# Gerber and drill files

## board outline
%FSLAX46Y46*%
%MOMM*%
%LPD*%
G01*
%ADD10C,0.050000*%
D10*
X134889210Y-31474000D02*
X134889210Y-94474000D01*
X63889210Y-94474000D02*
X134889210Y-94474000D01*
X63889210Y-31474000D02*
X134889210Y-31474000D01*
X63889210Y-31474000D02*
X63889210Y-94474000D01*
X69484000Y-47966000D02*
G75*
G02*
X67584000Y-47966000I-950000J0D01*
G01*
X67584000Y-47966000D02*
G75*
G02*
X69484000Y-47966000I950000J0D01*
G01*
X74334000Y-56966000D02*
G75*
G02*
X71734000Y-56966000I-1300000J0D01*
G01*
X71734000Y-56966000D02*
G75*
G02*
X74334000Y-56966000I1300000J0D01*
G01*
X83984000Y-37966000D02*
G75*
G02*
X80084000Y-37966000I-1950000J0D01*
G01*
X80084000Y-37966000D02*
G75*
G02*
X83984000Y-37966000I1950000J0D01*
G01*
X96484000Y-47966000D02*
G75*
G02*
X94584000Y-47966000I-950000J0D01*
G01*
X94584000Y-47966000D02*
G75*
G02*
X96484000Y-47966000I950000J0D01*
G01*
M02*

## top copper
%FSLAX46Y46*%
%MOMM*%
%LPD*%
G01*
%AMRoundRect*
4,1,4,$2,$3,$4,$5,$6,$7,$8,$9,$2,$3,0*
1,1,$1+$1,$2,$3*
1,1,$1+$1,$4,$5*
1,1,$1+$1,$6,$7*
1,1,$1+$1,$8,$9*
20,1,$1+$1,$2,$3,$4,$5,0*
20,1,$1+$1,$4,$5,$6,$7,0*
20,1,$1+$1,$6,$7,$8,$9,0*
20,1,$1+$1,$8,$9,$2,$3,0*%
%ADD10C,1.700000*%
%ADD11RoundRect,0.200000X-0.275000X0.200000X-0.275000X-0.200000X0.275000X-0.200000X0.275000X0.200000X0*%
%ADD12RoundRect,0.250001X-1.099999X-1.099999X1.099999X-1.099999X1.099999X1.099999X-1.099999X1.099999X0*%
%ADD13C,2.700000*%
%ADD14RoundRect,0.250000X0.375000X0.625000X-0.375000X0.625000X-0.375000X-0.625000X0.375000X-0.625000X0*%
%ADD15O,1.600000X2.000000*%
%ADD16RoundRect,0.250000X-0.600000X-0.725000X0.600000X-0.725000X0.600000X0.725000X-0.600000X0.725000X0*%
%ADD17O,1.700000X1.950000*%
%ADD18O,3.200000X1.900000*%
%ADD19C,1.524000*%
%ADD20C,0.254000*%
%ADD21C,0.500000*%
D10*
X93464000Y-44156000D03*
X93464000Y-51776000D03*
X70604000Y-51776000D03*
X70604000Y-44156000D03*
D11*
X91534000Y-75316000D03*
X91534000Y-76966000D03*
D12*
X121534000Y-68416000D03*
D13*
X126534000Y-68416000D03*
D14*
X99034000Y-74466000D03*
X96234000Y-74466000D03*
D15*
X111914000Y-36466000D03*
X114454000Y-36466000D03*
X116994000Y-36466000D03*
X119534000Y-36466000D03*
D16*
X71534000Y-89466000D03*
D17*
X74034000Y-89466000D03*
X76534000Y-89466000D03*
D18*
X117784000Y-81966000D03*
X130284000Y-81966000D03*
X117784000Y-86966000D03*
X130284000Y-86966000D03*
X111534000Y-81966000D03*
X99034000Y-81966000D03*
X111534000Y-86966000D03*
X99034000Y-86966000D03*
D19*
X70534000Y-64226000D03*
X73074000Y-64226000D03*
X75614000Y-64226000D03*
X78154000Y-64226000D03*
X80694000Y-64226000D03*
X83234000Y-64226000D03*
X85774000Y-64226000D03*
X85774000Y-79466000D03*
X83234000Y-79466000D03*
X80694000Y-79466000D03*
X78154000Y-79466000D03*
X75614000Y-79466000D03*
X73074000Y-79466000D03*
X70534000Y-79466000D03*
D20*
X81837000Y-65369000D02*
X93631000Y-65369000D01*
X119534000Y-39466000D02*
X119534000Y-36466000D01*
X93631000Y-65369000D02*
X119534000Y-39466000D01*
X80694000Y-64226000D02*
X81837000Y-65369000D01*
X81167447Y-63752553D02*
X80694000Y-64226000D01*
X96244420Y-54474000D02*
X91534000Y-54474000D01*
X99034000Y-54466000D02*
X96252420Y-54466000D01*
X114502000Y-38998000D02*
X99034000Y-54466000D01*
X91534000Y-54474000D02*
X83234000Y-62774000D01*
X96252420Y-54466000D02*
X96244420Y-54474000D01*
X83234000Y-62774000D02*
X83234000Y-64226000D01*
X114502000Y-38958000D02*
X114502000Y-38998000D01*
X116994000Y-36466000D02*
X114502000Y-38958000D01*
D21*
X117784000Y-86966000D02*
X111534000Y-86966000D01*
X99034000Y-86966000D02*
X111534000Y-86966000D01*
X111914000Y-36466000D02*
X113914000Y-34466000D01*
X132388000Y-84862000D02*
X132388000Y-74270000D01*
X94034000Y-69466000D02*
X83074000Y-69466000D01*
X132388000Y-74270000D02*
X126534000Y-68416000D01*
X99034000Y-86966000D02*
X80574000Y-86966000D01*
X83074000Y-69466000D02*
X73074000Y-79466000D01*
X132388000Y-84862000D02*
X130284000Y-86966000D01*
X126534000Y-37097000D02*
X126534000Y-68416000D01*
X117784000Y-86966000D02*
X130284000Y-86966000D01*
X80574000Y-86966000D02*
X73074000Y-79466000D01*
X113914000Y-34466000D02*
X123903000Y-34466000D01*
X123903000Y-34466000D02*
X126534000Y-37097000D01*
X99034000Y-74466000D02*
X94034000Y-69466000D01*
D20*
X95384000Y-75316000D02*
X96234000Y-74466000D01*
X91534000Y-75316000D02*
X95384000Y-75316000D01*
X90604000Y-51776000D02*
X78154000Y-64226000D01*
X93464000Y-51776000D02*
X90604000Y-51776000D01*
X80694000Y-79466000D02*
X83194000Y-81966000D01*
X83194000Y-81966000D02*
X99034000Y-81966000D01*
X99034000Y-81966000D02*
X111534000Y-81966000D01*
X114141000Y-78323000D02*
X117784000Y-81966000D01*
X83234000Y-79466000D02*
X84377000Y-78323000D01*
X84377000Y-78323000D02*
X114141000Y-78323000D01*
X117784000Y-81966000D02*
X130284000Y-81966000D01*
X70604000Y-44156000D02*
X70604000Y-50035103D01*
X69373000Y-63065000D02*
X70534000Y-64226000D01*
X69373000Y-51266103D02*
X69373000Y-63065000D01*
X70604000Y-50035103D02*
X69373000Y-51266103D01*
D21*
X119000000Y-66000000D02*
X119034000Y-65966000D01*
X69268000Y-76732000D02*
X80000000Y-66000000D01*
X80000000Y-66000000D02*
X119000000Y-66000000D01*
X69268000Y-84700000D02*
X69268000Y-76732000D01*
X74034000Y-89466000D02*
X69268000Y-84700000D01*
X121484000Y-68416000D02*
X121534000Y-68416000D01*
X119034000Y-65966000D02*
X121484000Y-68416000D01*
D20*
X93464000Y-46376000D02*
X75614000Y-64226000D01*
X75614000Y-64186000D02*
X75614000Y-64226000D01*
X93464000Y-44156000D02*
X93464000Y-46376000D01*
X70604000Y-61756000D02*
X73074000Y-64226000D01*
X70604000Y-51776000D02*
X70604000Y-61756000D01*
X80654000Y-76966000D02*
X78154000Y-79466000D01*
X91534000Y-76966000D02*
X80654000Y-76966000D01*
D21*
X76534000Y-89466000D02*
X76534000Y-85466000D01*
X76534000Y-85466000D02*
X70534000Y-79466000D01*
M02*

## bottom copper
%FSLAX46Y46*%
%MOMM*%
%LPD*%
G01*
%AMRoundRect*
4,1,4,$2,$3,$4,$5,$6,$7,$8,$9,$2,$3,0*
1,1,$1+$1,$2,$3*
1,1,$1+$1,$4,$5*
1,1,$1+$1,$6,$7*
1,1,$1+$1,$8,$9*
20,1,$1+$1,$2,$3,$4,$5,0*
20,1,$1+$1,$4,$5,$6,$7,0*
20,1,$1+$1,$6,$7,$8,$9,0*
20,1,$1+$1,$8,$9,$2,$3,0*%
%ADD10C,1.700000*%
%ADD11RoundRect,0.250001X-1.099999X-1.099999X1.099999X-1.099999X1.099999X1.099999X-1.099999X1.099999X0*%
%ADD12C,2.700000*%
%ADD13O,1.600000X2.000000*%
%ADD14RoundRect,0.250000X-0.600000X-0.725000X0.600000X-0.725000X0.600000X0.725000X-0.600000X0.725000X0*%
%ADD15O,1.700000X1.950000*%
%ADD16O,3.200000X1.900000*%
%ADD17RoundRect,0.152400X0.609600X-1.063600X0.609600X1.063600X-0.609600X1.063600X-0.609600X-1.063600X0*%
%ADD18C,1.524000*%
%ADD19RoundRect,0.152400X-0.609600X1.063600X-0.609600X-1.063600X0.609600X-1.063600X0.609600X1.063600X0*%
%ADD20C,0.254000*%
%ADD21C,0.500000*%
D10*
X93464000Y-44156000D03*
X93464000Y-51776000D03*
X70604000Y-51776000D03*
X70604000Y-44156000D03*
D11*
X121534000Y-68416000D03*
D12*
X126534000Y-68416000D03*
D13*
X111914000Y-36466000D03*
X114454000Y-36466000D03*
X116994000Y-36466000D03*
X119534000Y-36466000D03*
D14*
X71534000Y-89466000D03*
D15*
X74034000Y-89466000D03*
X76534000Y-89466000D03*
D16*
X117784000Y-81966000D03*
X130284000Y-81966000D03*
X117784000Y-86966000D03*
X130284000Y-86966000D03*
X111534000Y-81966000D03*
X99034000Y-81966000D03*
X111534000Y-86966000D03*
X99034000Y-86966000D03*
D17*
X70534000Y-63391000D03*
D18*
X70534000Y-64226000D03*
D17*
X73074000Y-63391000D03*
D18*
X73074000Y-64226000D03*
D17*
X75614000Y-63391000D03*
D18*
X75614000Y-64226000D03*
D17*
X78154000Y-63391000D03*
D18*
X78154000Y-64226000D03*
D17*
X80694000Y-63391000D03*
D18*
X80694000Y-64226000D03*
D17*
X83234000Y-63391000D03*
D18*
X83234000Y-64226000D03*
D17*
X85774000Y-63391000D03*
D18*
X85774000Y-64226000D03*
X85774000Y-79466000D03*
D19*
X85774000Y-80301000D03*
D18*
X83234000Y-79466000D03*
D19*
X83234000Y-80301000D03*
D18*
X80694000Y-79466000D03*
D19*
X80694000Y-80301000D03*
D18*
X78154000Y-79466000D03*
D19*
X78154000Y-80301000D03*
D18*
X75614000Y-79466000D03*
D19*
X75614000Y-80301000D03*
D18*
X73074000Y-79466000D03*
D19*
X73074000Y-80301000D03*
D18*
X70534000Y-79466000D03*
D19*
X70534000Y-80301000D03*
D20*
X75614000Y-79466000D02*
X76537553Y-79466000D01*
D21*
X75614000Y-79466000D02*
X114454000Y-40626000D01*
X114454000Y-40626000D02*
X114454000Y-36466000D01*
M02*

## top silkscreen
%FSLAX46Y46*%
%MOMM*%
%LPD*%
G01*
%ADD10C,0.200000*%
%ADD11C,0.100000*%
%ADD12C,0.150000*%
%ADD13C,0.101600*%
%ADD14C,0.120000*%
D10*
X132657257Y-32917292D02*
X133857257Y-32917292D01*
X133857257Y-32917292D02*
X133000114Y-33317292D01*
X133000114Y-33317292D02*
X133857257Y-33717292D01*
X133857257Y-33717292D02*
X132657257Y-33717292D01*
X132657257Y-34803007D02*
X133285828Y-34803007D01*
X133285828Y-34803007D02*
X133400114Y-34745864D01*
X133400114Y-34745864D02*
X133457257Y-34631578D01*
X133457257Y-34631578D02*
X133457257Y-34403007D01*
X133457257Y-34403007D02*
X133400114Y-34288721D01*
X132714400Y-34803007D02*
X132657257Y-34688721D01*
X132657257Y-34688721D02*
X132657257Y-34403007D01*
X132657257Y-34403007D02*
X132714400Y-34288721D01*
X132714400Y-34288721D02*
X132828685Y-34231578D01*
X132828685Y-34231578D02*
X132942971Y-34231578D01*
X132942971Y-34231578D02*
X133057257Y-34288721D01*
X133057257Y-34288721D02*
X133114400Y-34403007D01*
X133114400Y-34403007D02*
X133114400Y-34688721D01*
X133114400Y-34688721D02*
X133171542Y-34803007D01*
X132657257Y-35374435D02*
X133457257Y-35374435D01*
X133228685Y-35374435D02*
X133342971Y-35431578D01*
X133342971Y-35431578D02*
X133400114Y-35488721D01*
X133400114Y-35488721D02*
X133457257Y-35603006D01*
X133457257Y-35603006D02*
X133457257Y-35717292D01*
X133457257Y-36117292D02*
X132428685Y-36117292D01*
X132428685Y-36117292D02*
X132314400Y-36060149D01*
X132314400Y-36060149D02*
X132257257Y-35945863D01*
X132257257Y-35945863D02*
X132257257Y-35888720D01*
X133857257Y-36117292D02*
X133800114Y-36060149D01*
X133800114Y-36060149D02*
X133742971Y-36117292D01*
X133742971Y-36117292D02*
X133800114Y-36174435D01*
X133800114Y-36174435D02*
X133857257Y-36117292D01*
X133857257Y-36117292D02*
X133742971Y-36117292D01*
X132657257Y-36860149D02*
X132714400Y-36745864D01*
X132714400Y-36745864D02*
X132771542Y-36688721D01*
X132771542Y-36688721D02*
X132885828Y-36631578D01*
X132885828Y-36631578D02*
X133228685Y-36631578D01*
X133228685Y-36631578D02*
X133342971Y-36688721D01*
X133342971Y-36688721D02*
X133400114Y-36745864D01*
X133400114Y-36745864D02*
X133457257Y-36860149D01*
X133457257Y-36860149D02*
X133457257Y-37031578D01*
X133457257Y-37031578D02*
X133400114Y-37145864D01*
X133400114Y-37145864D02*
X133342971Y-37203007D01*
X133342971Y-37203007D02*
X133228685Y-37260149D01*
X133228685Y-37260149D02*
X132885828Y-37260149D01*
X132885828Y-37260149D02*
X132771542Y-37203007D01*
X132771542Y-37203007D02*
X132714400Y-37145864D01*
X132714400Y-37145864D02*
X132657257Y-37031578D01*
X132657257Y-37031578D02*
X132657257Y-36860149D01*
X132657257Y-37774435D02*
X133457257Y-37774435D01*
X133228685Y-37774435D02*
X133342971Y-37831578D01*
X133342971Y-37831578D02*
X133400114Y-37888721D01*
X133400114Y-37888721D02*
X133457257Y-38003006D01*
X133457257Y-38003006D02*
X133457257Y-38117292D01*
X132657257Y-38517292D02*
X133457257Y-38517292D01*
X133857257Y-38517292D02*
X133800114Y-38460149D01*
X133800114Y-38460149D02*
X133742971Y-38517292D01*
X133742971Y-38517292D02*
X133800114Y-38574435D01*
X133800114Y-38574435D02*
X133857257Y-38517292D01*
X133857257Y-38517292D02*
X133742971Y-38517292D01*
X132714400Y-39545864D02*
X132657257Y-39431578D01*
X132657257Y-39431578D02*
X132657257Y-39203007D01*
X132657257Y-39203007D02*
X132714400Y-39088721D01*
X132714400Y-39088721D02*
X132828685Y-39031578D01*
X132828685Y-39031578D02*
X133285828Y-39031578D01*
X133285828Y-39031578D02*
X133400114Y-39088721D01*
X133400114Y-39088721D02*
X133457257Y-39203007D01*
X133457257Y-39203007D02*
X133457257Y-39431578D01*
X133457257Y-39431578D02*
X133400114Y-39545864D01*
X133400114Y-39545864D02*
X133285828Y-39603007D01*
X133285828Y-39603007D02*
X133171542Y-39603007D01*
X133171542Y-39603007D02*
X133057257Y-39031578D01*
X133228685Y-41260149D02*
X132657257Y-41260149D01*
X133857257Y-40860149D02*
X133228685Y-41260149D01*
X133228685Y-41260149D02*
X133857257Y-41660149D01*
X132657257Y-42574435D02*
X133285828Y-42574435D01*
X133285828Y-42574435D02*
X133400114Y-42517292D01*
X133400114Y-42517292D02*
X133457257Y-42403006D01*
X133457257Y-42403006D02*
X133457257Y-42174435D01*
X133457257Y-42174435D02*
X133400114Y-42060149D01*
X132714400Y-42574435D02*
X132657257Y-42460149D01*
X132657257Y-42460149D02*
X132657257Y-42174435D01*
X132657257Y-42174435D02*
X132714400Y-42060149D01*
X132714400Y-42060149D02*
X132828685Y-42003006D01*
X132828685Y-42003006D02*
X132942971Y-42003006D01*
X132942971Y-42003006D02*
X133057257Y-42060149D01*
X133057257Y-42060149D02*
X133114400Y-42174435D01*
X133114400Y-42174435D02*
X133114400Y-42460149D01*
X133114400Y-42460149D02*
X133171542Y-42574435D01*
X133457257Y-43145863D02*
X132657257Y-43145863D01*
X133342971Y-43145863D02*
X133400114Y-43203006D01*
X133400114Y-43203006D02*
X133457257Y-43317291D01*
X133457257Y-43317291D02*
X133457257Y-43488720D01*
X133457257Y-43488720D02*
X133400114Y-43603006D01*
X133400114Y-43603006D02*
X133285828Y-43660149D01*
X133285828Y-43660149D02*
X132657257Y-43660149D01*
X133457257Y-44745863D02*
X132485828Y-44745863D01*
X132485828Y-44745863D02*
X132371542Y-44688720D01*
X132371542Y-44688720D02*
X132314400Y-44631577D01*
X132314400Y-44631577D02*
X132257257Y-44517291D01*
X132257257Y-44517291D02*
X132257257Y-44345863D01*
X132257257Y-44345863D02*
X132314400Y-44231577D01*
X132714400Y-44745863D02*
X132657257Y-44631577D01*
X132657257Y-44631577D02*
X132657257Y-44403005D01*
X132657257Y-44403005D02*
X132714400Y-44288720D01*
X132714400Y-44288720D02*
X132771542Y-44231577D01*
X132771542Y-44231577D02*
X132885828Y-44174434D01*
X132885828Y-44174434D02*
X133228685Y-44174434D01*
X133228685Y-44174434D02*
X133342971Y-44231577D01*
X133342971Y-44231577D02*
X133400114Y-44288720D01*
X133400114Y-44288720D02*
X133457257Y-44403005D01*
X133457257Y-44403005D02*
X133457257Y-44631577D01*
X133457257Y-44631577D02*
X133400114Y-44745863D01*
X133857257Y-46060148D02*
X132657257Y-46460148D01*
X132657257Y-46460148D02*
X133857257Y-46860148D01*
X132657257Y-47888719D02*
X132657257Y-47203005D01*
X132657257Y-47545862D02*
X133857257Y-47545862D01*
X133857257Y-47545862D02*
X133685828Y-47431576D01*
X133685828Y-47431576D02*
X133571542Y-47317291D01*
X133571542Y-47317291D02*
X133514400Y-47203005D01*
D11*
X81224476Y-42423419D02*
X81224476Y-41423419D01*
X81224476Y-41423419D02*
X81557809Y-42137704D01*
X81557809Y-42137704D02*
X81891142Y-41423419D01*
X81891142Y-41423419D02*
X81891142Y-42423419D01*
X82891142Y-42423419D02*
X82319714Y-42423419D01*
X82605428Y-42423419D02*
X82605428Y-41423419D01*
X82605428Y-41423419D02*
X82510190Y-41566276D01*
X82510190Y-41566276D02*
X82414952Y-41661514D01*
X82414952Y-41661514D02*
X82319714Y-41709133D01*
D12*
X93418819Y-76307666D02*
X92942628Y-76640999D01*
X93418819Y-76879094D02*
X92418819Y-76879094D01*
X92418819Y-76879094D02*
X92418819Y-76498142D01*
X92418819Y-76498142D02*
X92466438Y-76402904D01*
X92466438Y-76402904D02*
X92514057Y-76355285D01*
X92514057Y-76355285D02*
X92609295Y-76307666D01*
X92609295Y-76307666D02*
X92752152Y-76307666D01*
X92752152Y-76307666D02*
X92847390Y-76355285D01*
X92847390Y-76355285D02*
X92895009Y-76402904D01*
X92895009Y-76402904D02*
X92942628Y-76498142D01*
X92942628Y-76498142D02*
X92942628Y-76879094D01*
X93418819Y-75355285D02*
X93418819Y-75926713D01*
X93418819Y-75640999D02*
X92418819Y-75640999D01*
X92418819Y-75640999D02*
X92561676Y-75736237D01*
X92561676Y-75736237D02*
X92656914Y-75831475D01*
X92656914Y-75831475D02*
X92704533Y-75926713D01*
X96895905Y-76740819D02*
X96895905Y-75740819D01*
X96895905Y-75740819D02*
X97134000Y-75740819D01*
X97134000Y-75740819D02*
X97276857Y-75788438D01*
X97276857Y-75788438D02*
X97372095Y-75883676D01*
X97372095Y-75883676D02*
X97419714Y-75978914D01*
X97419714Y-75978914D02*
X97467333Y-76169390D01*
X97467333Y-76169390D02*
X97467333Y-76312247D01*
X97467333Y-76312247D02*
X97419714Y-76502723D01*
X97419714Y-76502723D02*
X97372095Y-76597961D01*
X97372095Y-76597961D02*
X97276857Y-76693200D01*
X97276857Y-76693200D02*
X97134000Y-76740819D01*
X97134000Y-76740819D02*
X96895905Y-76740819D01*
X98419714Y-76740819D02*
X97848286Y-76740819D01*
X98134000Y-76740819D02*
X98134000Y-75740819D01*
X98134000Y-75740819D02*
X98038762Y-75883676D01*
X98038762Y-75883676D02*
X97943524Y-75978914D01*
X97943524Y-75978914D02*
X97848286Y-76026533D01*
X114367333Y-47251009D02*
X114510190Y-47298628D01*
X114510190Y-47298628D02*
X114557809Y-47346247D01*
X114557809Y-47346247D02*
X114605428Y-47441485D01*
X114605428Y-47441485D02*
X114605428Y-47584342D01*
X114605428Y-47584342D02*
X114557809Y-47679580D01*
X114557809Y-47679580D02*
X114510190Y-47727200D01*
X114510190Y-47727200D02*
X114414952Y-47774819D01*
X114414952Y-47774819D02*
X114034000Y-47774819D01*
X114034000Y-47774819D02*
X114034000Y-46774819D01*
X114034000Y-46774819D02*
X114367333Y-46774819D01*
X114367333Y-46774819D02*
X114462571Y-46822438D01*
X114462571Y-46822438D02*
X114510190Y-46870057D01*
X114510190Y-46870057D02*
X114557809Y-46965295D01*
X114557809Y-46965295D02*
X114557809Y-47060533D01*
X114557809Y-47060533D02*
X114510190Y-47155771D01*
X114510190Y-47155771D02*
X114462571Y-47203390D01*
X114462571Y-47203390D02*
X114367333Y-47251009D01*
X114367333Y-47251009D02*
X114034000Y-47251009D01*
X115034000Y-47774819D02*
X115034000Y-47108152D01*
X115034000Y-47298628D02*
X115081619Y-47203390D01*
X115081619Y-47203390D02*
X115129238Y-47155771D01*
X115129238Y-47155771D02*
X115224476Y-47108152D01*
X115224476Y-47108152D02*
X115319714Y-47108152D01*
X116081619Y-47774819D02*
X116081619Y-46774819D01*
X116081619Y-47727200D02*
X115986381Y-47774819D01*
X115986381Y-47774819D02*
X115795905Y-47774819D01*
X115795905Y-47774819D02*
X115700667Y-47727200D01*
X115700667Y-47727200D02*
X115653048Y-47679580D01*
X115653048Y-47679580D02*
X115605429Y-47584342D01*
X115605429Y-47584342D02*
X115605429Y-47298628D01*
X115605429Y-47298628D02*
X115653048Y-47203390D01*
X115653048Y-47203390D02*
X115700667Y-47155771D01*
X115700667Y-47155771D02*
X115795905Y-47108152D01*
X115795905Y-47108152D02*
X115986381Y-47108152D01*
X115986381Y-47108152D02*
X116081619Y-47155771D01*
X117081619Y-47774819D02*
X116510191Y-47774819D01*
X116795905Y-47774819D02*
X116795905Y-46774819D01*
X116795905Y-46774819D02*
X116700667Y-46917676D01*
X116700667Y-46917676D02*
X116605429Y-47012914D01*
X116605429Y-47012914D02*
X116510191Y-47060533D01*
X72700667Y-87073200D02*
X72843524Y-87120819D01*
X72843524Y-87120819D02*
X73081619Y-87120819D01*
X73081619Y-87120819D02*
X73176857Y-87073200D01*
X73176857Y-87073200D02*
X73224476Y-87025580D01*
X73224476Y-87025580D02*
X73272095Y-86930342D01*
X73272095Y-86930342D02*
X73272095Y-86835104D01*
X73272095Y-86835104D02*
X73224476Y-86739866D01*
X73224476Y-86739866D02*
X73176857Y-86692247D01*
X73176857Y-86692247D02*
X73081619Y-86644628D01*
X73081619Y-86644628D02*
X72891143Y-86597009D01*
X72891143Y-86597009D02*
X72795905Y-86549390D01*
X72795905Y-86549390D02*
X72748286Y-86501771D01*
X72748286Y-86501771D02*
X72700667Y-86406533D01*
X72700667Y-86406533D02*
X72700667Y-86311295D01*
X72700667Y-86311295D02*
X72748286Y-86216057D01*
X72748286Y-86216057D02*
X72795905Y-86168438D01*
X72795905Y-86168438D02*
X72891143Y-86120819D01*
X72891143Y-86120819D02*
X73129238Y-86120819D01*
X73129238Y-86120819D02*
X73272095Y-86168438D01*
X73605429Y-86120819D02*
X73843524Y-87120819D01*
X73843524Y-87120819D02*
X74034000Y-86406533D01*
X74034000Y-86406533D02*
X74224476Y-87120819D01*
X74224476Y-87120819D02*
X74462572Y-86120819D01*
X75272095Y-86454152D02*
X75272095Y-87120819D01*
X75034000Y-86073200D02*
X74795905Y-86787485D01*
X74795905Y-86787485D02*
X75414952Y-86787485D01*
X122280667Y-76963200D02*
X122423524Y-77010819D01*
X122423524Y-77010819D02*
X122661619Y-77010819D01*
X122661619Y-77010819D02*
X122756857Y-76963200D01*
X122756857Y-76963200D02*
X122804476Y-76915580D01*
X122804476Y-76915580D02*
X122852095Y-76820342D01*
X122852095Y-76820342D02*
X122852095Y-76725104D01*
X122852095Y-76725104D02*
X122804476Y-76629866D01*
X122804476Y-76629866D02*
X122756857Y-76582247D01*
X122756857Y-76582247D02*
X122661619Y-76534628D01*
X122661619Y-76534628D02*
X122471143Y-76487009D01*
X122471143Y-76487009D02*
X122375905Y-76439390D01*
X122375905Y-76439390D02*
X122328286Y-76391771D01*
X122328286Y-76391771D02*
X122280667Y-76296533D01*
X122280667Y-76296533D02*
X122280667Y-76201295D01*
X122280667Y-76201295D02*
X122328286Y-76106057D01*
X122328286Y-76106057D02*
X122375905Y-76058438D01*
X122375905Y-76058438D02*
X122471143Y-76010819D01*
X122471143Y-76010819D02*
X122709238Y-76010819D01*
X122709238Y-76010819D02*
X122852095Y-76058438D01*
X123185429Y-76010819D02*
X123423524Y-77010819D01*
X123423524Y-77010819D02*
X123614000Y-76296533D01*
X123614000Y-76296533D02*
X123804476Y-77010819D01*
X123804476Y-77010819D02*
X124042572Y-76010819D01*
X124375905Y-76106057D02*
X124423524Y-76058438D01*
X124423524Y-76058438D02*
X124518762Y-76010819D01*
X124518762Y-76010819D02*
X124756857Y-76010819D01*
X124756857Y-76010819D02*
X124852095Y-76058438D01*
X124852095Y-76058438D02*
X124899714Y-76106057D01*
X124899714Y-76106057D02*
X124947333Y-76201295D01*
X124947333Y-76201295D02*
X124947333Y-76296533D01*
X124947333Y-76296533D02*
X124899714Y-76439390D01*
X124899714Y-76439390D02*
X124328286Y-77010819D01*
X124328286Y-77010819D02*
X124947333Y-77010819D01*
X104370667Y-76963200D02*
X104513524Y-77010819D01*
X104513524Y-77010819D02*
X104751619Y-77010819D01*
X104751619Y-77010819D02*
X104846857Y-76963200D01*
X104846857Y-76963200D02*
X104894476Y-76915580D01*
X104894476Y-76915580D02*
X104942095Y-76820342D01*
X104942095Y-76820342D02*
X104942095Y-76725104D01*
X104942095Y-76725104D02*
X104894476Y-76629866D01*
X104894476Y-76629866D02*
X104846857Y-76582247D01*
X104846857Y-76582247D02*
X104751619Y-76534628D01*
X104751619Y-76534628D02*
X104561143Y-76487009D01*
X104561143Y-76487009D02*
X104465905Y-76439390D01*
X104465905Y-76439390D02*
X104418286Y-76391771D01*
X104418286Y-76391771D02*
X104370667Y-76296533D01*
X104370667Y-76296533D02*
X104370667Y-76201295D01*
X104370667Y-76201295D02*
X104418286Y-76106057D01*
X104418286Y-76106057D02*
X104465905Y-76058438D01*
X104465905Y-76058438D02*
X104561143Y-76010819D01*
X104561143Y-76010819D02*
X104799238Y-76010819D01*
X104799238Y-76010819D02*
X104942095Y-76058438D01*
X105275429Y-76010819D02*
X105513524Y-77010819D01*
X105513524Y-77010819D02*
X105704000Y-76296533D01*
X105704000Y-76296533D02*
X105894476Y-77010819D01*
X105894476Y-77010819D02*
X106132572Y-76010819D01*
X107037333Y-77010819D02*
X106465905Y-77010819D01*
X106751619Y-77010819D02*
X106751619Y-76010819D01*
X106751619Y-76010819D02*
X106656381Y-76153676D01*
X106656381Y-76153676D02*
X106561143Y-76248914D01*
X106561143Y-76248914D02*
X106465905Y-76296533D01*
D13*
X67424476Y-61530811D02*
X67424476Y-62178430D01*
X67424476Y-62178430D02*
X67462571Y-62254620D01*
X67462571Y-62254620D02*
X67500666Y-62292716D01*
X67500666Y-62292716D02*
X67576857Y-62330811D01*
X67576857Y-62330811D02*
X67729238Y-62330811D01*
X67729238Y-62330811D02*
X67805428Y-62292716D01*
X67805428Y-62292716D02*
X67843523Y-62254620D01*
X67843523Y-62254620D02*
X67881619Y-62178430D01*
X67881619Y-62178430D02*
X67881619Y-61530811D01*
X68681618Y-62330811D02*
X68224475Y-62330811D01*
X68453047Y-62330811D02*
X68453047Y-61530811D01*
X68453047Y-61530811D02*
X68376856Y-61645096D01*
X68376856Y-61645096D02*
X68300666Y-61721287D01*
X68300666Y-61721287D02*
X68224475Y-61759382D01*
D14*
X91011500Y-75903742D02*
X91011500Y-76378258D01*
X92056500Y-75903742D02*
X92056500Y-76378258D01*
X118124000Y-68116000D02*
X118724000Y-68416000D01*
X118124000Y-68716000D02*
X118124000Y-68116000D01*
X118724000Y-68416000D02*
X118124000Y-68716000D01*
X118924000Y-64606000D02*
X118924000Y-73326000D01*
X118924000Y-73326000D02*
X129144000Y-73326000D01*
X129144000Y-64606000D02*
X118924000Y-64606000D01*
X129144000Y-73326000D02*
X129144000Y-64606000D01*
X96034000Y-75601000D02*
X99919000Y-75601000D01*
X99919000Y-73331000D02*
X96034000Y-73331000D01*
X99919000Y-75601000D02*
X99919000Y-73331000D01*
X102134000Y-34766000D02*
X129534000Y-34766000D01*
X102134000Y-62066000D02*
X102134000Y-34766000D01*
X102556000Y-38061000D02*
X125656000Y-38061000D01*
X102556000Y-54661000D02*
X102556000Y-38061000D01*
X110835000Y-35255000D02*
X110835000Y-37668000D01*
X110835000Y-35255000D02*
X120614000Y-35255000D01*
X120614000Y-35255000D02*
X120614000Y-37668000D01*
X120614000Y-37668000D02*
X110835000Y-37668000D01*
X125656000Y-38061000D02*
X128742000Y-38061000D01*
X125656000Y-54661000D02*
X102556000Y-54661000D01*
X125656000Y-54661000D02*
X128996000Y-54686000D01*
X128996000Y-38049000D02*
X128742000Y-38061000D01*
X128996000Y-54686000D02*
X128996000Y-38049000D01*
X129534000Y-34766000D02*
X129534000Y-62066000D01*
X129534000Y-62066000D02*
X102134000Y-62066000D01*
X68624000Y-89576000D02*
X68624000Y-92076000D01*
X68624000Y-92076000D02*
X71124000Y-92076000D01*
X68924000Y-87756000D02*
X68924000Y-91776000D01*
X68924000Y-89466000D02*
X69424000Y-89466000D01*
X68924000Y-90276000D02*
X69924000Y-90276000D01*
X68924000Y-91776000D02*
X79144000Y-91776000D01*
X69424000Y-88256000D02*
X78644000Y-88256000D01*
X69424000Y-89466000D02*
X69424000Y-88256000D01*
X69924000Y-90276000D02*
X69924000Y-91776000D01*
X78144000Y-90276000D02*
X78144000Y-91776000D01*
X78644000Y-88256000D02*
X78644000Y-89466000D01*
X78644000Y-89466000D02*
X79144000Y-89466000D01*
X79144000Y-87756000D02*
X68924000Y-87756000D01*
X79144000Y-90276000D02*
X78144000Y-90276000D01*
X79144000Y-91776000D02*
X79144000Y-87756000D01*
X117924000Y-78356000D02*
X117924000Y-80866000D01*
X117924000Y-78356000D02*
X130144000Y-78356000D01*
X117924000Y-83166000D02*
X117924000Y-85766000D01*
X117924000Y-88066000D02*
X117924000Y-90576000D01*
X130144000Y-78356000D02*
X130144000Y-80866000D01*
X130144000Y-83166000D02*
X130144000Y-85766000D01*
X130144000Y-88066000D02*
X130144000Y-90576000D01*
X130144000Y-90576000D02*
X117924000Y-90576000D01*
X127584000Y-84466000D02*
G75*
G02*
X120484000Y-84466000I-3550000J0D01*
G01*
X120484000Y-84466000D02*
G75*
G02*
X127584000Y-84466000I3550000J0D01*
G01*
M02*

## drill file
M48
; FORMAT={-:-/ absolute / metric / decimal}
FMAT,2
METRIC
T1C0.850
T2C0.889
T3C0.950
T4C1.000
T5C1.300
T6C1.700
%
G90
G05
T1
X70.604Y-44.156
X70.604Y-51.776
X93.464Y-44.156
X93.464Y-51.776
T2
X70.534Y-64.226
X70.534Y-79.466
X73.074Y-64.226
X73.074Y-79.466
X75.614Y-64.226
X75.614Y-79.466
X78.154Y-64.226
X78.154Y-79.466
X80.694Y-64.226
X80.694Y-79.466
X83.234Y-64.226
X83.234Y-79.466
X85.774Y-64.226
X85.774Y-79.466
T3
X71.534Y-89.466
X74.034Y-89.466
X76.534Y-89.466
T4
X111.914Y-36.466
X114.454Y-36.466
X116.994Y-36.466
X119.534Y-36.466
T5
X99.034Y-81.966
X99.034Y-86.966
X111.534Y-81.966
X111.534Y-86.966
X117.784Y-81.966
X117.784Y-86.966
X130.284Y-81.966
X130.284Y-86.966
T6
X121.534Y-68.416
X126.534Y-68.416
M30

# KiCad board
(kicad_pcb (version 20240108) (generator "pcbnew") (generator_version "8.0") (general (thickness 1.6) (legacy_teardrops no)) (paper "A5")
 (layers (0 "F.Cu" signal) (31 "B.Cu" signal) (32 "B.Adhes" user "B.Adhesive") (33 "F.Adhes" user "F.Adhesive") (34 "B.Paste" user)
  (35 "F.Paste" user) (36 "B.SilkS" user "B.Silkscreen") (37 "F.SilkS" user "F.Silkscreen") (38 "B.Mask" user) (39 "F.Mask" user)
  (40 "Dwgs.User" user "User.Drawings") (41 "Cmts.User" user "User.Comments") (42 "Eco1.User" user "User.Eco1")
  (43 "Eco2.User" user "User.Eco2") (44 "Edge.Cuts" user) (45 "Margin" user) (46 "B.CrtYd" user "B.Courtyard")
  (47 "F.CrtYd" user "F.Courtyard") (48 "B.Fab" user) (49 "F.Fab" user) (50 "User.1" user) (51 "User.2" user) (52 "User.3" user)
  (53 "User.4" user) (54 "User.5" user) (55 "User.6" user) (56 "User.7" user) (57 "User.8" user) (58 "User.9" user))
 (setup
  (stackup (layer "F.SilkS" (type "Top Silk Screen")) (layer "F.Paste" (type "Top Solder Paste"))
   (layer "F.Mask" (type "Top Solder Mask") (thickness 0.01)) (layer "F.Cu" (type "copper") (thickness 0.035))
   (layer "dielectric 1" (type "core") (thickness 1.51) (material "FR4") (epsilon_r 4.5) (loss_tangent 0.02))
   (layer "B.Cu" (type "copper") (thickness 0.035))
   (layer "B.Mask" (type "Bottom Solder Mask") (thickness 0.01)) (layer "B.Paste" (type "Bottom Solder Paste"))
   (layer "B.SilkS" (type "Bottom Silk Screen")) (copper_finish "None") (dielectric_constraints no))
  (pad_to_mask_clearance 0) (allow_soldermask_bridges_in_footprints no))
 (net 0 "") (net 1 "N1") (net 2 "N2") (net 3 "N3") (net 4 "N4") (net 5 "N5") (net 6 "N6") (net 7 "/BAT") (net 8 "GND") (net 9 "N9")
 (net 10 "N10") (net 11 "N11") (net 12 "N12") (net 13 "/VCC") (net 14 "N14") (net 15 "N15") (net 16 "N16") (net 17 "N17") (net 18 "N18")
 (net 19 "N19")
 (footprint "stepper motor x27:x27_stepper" (layer "F.Cu") (at 84.574 58.126)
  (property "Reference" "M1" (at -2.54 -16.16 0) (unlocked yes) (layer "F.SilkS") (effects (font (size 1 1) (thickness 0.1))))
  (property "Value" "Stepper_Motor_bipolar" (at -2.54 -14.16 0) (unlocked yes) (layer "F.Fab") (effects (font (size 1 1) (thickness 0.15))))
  (fp_circle (center -16.04 -10.16) (end -15.09 -10.16) (stroke (width 0.05) (type default)) (fill none) (layer "Edge.Cuts"))
  (fp_circle (center -11.54 -1.16) (end -10.24 -1.16) (stroke (width 0.05) (type default)) (fill none) (layer "Edge.Cuts"))
  (fp_circle (center -2.54 -20.16) (end -0.59 -20.16) (stroke (width 0.05) (type default)) (fill none) (layer "Edge.Cuts"))
  (fp_circle (center 10.96 -10.16) (end 11.91 -10.16) (stroke (width 0.05) (type default)) (fill none) (layer "Edge.Cuts"))
  (pad "1" thru_hole circle (at 8.89 -13.97) (size 1.7 1.7) (drill 0.85) (layers "*.Cu" "*.Mask") (remove_unused_layers no) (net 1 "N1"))
  (pad "2" thru_hole circle (at 8.89 -6.35) (size 1.7 1.7) (drill 0.85) (layers "*.Cu" "*.Mask") (remove_unused_layers no) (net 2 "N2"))
  (pad "3" thru_hole circle (at -13.97 -6.35) (size 1.7 1.7) (drill 0.85) (layers "*.Cu" "*.Mask") (remove_unused_layers no) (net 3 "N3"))
  (pad "4" thru_hole circle (at -13.97 -13.97) (size 1.7 1.7) (drill 0.85) (layers "*.Cu" "*.Mask") (remove_unused_layers no) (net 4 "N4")))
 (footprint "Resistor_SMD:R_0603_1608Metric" (layer "F.Cu") (at 91.534 76.141 -90)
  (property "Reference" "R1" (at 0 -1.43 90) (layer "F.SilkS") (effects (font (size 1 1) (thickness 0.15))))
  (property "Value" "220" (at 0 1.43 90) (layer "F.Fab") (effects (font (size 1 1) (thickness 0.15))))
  (fp_line (start -0.237258 0.5225) (end 0.237258 0.5225) (stroke (width 0.12) (type solid)) (layer "F.SilkS"))
  (fp_line (start -0.237258 -0.5225) (end 0.237258 -0.5225) (stroke (width 0.12) (type solid)) (layer "F.SilkS"))
  (pad "1" smd roundrect (at -0.825 0 270) (size 0.8 0.95) (layers "F.Cu" "F.Paste" "F.Mask") (roundrect_rratio 0.25) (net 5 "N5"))
  (pad "2" smd roundrect (at 0.825 0 270) (size 0.8 0.95) (layers "F.Cu" "F.Paste" "F.Mask") (roundrect_rratio 0.25) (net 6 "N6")))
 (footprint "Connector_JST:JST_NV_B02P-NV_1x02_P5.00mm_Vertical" (layer "F.Cu") (at 121.534 68.416)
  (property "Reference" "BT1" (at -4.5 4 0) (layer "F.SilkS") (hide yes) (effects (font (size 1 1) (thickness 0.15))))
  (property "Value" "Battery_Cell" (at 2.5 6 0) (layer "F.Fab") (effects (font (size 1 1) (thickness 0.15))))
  (fp_line (start -3.41 -0.3) (end -2.81 0) (stroke (width 0.12) (type solid)) (layer "F.SilkS"))
  (fp_line (start -3.41 0.3) (end -3.41 -0.3) (stroke (width 0.12) (type solid)) (layer "F.SilkS"))
  (fp_line (start -2.81 0) (end -3.41 0.3) (stroke (width 0.12) (type solid)) (layer "F.SilkS"))
  (fp_line (start -2.61 -3.81) (end -2.61 4.91) (stroke (width 0.12) (type solid)) (layer "F.SilkS"))
  (fp_line (start -2.61 4.91) (end 7.61 4.91) (stroke (width 0.12) (type solid)) (layer "F.SilkS"))
  (fp_line (start 7.61 -3.81) (end -2.61 -3.81) (stroke (width 0.12) (type solid)) (layer "F.SilkS"))
  (fp_line (start 7.61 4.91) (end 7.61 -3.81) (stroke (width 0.12) (type solid)) (layer "F.SilkS"))
  (pad "1" thru_hole roundrect (at 0 0) (size 2.7 2.7) (drill 1.7) (layers "*.Cu" "*.Mask") (remove_unused_layers no)
   (roundrect_rratio 0.092593) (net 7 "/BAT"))
  (pad "2" thru_hole circle (at 5 0) (size 2.7 2.7) (drill 1.7) (layers "*.Cu" "*.Mask") (remove_unused_layers no) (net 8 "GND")))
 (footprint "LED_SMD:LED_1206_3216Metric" (layer "F.Cu") (at 97.634 74.466 180)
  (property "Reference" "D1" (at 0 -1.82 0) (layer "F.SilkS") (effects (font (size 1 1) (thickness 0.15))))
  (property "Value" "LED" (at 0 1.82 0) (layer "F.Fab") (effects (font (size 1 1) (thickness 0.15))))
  (fp_line (start 1.6 -1.135) (end -2.285 -1.135) (stroke (width 0.12) (type solid)) (layer "F.SilkS"))
  (fp_line (start -2.285 1.135) (end 1.6 1.135) (stroke (width 0.12) (type solid)) (layer "F.SilkS"))
  (fp_line (start -2.285 -1.135) (end -2.285 1.135) (stroke (width 0.12) (type solid)) (layer "F.SilkS"))
  (pad "1" smd roundrect (at -1.4 0 180) (size 1.25 1.75) (layers "F.Cu" "F.Paste" "F.Mask") (roundrect_rratio 0.2) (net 8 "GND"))
  (pad "2" smd roundrect (at 1.4 0 180) (size 1.25 1.75) (layers "F.Cu" "F.Paste" "F.Mask") (roundrect_rratio 0.2) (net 5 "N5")))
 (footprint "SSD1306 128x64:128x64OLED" (layer "F.Cu") (at 115.534 47.066)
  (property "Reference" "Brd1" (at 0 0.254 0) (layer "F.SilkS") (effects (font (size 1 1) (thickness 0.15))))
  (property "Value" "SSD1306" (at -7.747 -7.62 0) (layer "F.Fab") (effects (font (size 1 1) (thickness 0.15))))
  (fp_line (start -13.4 -12.3) (end 14 -12.3) (stroke (width 0.12) (type solid)) (layer "F.SilkS"))
  (fp_line (start -13.4 15) (end -13.4 -12.3) (stroke (width 0.12) (type solid)) (layer "F.SilkS"))
  (fp_line (start -12.978 -9.005) (end 10.122 -9.005) (stroke (width 0.12) (type solid)) (layer "F.SilkS"))
  (fp_line (start -12.978 7.595) (end -12.978 -9.005) (stroke (width 0.12) (type solid)) (layer "F.SilkS"))
  (fp_line (start -4.699 -11.811) (end -4.699 -9.398) (stroke (width 0.12) (type solid)) (layer "F.SilkS"))
  (fp_line (start -4.699 -11.811) (end 5.08 -11.811) (stroke (width 0.12) (type solid)) (layer "F.SilkS"))
  (fp_line (start 5.08 -11.811) (end 5.08 -9.398) (stroke (width 0.12) (type solid)) (layer "F.SilkS"))
  (fp_line (start 5.08 -9.398) (end -4.699 -9.398) (stroke (width 0.12) (type solid)) (layer "F.SilkS"))
  (fp_line (start 10.122 -9.005) (end 13.208 -9.005) (stroke (width 0.12) (type solid)) (layer "F.SilkS"))
  (fp_line (start 10.122 7.595) (end -12.978 7.595) (stroke (width 0.12) (type solid)) (layer "F.SilkS"))
  (fp_line (start 10.122 7.595) (end 13.462 7.62) (stroke (width 0.12) (type solid)) (layer "F.SilkS"))
  (fp_line (start 13.462 -9.017) (end 13.208 -9.005) (stroke (width 0.12) (type solid)) (layer "F.SilkS"))
  (fp_line (start 13.462 7.62) (end 13.462 -9.017) (stroke (width 0.12) (type solid)) (layer "F.SilkS"))
  (fp_line (start 14 -12.3) (end 14 15) (stroke (width 0.12) (type solid)) (layer "F.SilkS"))
  (fp_line (start 14 15) (end -13.4 15) (stroke (width 0.12) (type solid)) (layer "F.SilkS"))
  (pad "1" thru_hole oval (at -3.62 -10.6 90) (size 2 1.6) (drill 1) (layers "*.Cu" "*.Mask") (remove_unused_layers no) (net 8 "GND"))
  (pad "2" thru_hole oval (at -1.08 -10.6 90) (size 2 1.6) (drill 1) (layers "*.Cu" "*.Mask") (remove_unused_layers no) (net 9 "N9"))
  (pad "3" thru_hole oval (at 1.46 -10.6 90) (size 2 1.6) (drill 1) (layers "*.Cu" "*.Mask") (remove_unused_layers no) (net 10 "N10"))
  (pad "4" thru_hole oval (at 4 -10.6 90) (size 2 1.6) (drill 1) (layers "*.Cu" "*.Mask") (remove_unused_layers no) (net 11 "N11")))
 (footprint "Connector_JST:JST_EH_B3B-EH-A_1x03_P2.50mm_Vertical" (layer "F.Cu") (at 71.534 89.466)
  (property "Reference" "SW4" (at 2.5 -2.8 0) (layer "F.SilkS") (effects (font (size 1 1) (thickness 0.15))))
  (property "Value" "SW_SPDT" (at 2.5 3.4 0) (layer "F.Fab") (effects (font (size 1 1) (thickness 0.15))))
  (fp_line (start -2.91 0.11) (end -2.91 2.61) (stroke (width 0.12) (type solid)) (layer "F.SilkS"))
  (fp_line (start -2.91 2.61) (end -0.41 2.61) (stroke (width 0.12) (type solid)) (layer "F.SilkS"))
  (fp_line (start -2.61 -1.71) (end -2.61 2.31) (stroke (width 0.12) (type solid)) (layer "F.SilkS"))
  (fp_line (start -2.61 0) (end -2.11 0) (stroke (width 0.12) (type solid)) (layer "F.SilkS"))
  (fp_line (start -2.61 0.81) (end -1.61 0.81) (stroke (width 0.12) (type solid)) (layer "F.SilkS"))
  (fp_line (start -2.61 2.31) (end 7.61 2.31) (stroke (width 0.12) (type solid)) (layer "F.SilkS"))
  (fp_line (start -2.11 -1.21) (end 7.11 -1.21) (stroke (width 0.12) (type solid)) (layer "F.SilkS"))
  (fp_line (start -2.11 0) (end -2.11 -1.21) (stroke (width 0.12) (type solid)) (layer "F.SilkS"))
  (fp_line (start -1.61 0.81) (end -1.61 2.31) (stroke (width 0.12) (type solid)) (layer "F.SilkS"))
  (fp_line (start 6.61 0.81) (end 6.61 2.31) (stroke (width 0.12) (type solid)) (layer "F.SilkS"))
  (fp_line (start 7.11 -1.21) (end 7.11 0) (stroke (width 0.12) (type solid)) (layer "F.SilkS"))
  (fp_line (start 7.11 0) (end 7.61 0) (stroke (width 0.12) (type solid)) (layer "F.SilkS"))
  (fp_line (start 7.61 -1.71) (end -2.61 -1.71) (stroke (width 0.12) (type solid)) (layer "F.SilkS"))
  (fp_line (start 7.61 0.81) (end 6.61 0.81) (stroke (width 0.12) (type solid)) (layer "F.SilkS"))
  (fp_line (start 7.61 2.31) (end 7.61 -1.71) (stroke (width 0.12) (type solid)) (layer "F.SilkS"))
  (pad "1" thru_hole roundrect (at 0 0) (size 1.7 1.95) (drill 0.95) (layers "*.Cu" "*.Mask") (remove_unused_layers no)
   (roundrect_rratio 0.147059) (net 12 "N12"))
  (pad "2" thru_hole oval (at 2.5 0) (size 1.7 1.95) (drill 0.95) (layers "*.Cu" "*.Mask") (remove_unused_layers no) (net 7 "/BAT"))
  (pad "3" thru_hole oval (at 5 0) (size 1.7 1.95) (drill 0.95) (layers "*.Cu" "*.Mask") (remove_unused_layers no) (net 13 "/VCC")))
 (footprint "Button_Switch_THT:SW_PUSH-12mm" (layer "F.Cu") (at 117.784 81.966)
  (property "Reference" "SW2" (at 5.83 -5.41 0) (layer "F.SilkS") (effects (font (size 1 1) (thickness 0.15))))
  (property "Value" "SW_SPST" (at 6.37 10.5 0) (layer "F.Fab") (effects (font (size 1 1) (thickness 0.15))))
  (fp_line (start 0.14 -3.61) (end 0.14 -1.1) (stroke (width 0.12) (type default)) (layer "F.SilkS"))
  (fp_line (start 0.14 -3.61) (end 12.36 -3.61) (stroke (width 0.12) (type default)) (layer "F.SilkS"))
  (fp_line (start 0.14 1.2) (end 0.14 3.8) (stroke (width 0.12) (type default)) (layer "F.SilkS"))
  (fp_line (start 0.14 6.1) (end 0.14 8.61) (stroke (width 0.12) (type default)) (layer "F.SilkS"))
  (fp_line (start 12.36 -3.61) (end 12.36 -1.1) (stroke (width 0.12) (type default)) (layer "F.SilkS"))
  (fp_line (start 12.36 1.2) (end 12.36 3.8) (stroke (width 0.12) (type default)) (layer "F.SilkS"))
  (fp_line (start 12.36 6.1) (end 12.36 8.61) (stroke (width 0.12) (type default)) (layer "F.SilkS"))
  (fp_line (start 12.36 8.61) (end 0.14 8.61) (stroke (width 0.12) (type default)) (layer "F.SilkS"))
  (fp_circle (center 6.25 2.5) (end 9.8 2.5) (stroke (width 0.12) (type default)) (fill none) (layer "F.SilkS"))
  (pad "1" thru_hole oval (at 0 0) (size 3.2 1.9) (drill 1.3) (layers "*.Cu" "*.Mask") (remove_unused_layers no) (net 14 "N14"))
  (pad "1" thru_hole oval (at 12.5 0) (size 3.2 1.9) (drill 1.3) (layers "*.Cu" "*.Mask") (remove_unused_layers no) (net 14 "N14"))
  (pad "2" thru_hole oval (at 0 5) (size 3.2 1.9) (drill 1.3) (layers "*.Cu" "*.Mask") (remove_unused_layers no) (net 8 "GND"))
  (pad "2" thru_hole oval (at 12.5 5) (size 3.2 1.9) (drill 1.3) (layers "*.Cu" "*.Mask") (remove_unused_layers no) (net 8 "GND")))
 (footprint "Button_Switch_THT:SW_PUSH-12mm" (layer "B.Cu") (at 111.534 81.966 180)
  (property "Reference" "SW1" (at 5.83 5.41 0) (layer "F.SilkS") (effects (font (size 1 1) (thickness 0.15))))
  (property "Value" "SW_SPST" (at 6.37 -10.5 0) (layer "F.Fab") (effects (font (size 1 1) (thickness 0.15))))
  (pad "1" thru_hole oval (at 0 0 180) (size 3.2 1.9) (drill 1.3) (layers "*.Cu" "*.Mask") (remove_unused_layers no) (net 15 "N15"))
  (pad "1" thru_hole oval (at 12.5 0 180) (size 3.2 1.9) (drill 1.3) (layers "*.Cu" "*.Mask") (remove_unused_layers no) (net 15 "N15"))
  (pad "2" thru_hole oval (at 0 -5 180) (size 3.2 1.9) (drill 1.3) (layers "*.Cu" "*.Mask") (remove_unused_layers no) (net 8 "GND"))
  (pad "2" thru_hole oval (at 12.5 -5 180) (size 3.2 1.9) (drill 1.3) (layers "*.Cu" "*.Mask") (remove_unused_layers no) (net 8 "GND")))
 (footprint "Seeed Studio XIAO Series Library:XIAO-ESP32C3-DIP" (layer "B.Cu") (at 78.154 71.966 -90)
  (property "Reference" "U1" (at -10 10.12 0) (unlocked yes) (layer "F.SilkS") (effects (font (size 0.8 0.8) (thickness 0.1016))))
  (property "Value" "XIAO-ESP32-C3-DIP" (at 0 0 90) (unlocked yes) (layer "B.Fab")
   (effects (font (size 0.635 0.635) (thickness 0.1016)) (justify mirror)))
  (pad "1" smd roundrect (at -8.575 7.62 90) (size 2.432 1.524) (layers "B.Cu" "B.Mask") (roundrect_rratio 0.1) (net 4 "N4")
   (thermal_bridge_angle 45))
  (pad "1" thru_hole circle (at -7.74 7.62 90) (size 1.524 1.524) (drill 0.889) (layers "*.Cu" "*.Mask") (remove_unused_layers no)
   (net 4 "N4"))
  (pad "2" smd roundrect (at -8.575 5.08 90) (size 2.432 1.524) (layers "B.Cu" "B.Mask") (roundrect_rratio 0.1) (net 3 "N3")
   (thermal_bridge_angle 45))
  (pad "2" thru_hole circle (at -7.74 5.08 90) (size 1.524 1.524) (drill 0.889) (layers "*.Cu" "*.Mask") (remove_unused_layers no)
   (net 3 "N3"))
  (pad "3" smd roundrect (at -8.575 2.54 90) (size 2.432 1.524) (layers "B.Cu" "B.Mask") (roundrect_rratio 0.1) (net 1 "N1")
   (thermal_bridge_angle 45))
  (pad "3" thru_hole circle (at -7.74 2.54 90) (size 1.524 1.524) (drill 0.889) (layers "*.Cu" "*.Mask") (remove_unused_layers no)
   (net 1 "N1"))
  (pad "4" smd roundrect (at -8.575 0 90) (size 2.432 1.524) (layers "B.Cu" "B.Mask") (roundrect_rratio 0.1) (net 2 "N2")
   (thermal_bridge_angle 45))
  (pad "4" thru_hole circle (at -7.74 0 90) (size 1.524 1.524) (drill 0.889) (layers "*.Cu" "*.Mask") (remove_unused_layers no) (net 2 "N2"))
  (pad "5" smd roundrect (at -8.575 -2.54 90) (size 2.432 1.524) (layers "B.Cu" "B.Mask") (roundrect_rratio 0.1) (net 11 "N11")
   (thermal_bridge_angle 45))
  (pad "5" thru_hole circle (at -7.74 -2.54 90) (size 1.524 1.524) (drill 0.889) (layers "*.Cu" "*.Mask") (remove_unused_layers no)
   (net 11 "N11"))
  (pad "6" smd roundrect (at -8.575 -5.08 90) (size 2.432 1.524) (layers "B.Cu" "B.Mask") (roundrect_rratio 0.1) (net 10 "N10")
   (thermal_bridge_angle 45))
  (pad "6" thru_hole circle (at -7.74 -5.08 90) (size 1.524 1.524) (drill 0.889) (layers "*.Cu" "*.Mask") (remove_unused_layers no)
   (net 10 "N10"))
  (pad "7" smd roundrect (at -8.575 -7.62 90) (size 2.432 1.524) (layers "B.Cu" "B.Mask") (roundrect_rratio 0.1) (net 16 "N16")
   (thermal_bridge_angle 45))
  (pad "7" thru_hole circle (at -7.74 -7.62 90) (size 1.524 1.524) (drill 0.889) (layers "*.Cu" "*.Mask") (remove_unused_layers no)
   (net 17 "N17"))
  (pad "8" thru_hole circle (at 7.5 -7.62 270) (size 1.524 1.524) (drill 0.889) (layers "*.Cu" "*.Mask") (remove_unused_layers no)
   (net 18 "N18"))
  (pad "8" smd roundrect (at 8.335 -7.62 270) (size 2.432 1.524) (layers "B.Cu" "B.Mask") (roundrect_rratio 0.1) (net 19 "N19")
   (thermal_bridge_angle 45))
  (pad "9" thru_hole circle (at 7.5 -5.08 270) (size 1.524 1.524) (drill 0.889) (layers "*.Cu" "*.Mask") (remove_unused_layers no)
   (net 14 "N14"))
  (pad "9" smd roundrect (at 8.335 -5.08 270) (size 2.432 1.524) (layers "B.Cu" "B.Mask") (roundrect_rratio 0.1) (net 14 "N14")
   (thermal_bridge_angle 45))
  (pad "10" thru_hole circle (at 7.5 -2.54 270) (size 1.524 1.524) (drill 0.889) (layers "*.Cu" "*.Mask") (remove_unused_layers no)
   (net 15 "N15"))
  (pad "10" smd roundrect (at 8.335 -2.54 270) (size 2.432 1.524) (layers "B.Cu" "B.Mask") (roundrect_rratio 0.1) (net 15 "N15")
   (thermal_bridge_angle 45))
  (pad "11" thru_hole circle (at 7.5 0 270) (size 1.524 1.524) (drill 0.889) (layers "*.Cu" "*.Mask") (remove_unused_layers no) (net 6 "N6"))
  (pad "11" smd roundrect (at 8.335 0 270) (size 2.432 1.524) (layers "B.Cu" "B.Mask") (roundrect_rratio 0.1) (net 6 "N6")
   (thermal_bridge_angle 45))
  (pad "12" thru_hole circle (at 7.5 2.54 270) (size 1.524 1.524) (drill 0.889) (layers "*.Cu" "*.Mask") (remove_unused_layers no)
   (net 9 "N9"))
  (pad "12" smd roundrect (at 8.335 2.54 270) (size 2.432 1.524) (layers "B.Cu" "B.Mask") (roundrect_rratio 0.1) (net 9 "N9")
   (thermal_bridge_angle 45))
  (pad "13" thru_hole circle (at 7.5 5.08 270) (size 1.524 1.524) (drill 0.889) (layers "*.Cu" "*.Mask") (remove_unused_layers no)
   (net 8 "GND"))
  (pad "13" smd roundrect (at 8.335 5.08 270) (size 2.432 1.524) (layers "B.Cu" "B.Mask") (roundrect_rratio 0.1) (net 8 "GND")
   (thermal_bridge_angle 45))
  (pad "14" thru_hole circle (at 7.5 7.62 270) (size 1.524 1.524) (drill 0.889) (layers "*.Cu" "*.Mask") (remove_unused_layers no)
   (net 13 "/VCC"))
  (pad "14" smd roundrect (at 8.335 7.62 270) (size 2.432 1.524) (layers "B.Cu" "B.Mask") (roundrect_rratio 0.1) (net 13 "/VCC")
   (thermal_bridge_angle 45)))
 (gr_line (start 134.88921 31.474) (end 134.88921 94.474) (stroke (width 0.05) (type default)) (layer "Edge.Cuts"))
 (gr_line (start 63.88921 94.474) (end 134.88921 94.474) (stroke (width 0.05) (type default)) (layer "Edge.Cuts"))
 (gr_line (start 63.88921 31.474) (end 134.88921 31.474) (stroke (width 0.05) (type default)) (layer "Edge.Cuts"))
 (gr_line (start 63.88921 31.474) (end 63.88921 94.474) (stroke (width 0.05) (type default)) (layer "Edge.Cuts"))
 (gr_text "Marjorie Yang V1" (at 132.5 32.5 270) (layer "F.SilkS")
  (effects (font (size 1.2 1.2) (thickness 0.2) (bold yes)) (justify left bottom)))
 (segment (start 81.837 65.369) (end 93.631 65.369) (width 0.254) (layer "F.Cu") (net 11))
 (segment (start 119.534 39.466) (end 119.534 36.466) (width 0.254) (layer "F.Cu") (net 11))
 (segment (start 93.631 65.369) (end 119.534 39.466) (width 0.254) (layer "F.Cu") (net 11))
 (segment (start 80.694 64.226) (end 81.837 65.369) (width 0.254) (layer "F.Cu") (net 11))
 (segment (start 81.167447 63.752553) (end 80.694 64.226) (width 0.254) (layer "F.Cu") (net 11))
 (segment (start 96.24442 54.474) (end 91.534 54.474) (width 0.254) (layer "F.Cu") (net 10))
 (segment (start 99.034 54.466) (end 96.25242 54.466) (width 0.254) (layer "F.Cu") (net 10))
 (segment (start 114.502 38.998) (end 99.034 54.466) (width 0.254) (layer "F.Cu") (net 10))
 (segment (start 91.534 54.474) (end 83.234 62.774) (width 0.254) (layer "F.Cu") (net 10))
 (segment (start 96.25242 54.466) (end 96.24442 54.474) (width 0.254) (layer "F.Cu") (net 10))
 (segment (start 83.234 62.774) (end 83.234 64.226) (width 0.254) (layer "F.Cu") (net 10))
 (segment (start 114.502 38.958) (end 114.502 38.998) (width 0.254) (layer "F.Cu") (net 10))
 (segment (start 116.994 36.466) (end 114.502 38.958) (width 0.254) (layer "F.Cu") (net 10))
 (segment (start 117.784 86.966) (end 111.534 86.966) (width 0.5) (layer "F.Cu") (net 8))
 (segment (start 99.034 86.966) (end 111.534 86.966) (width 0.5) (layer "F.Cu") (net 8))
 (segment (start 111.914 36.466) (end 113.914 34.466) (width 0.5) (layer "F.Cu") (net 8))
 (segment (start 132.388 84.862) (end 132.388 74.27) (width 0.5) (layer "F.Cu") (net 8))
 (segment (start 94.034 69.466) (end 83.074 69.466) (width 0.5) (layer "F.Cu") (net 8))
 (segment (start 132.388 74.27) (end 126.534 68.416) (width 0.5) (layer "F.Cu") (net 8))
 (segment (start 99.034 86.966) (end 80.574 86.966) (width 0.5) (layer "F.Cu") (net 8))
 (segment (start 83.074 69.466) (end 73.074 79.466) (width 0.5) (layer "F.Cu") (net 8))
 (segment (start 132.388 84.862) (end 130.284 86.966) (width 0.5) (layer "F.Cu") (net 8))
 (segment (start 126.534 37.097) (end 126.534 68.416) (width 0.5) (layer "F.Cu") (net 8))
 (segment (start 117.784 86.966) (end 130.284 86.966) (width 0.5) (layer "F.Cu") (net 8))
 (segment (start 80.574 86.966) (end 73.074 79.466) (width 0.5) (layer "F.Cu") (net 8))
 (segment (start 113.914 34.466) (end 123.903 34.466) (width 0.5) (layer "F.Cu") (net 8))
 (segment (start 123.903 34.466) (end 126.534 37.097) (width 0.5) (layer "F.Cu") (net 8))
 (segment (start 99.034 74.466) (end 94.034 69.466) (width 0.5) (layer "F.Cu") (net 8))
 (segment (start 95.384 75.316) (end 96.234 74.466) (width 0.254) (layer "F.Cu") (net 5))
 (segment (start 91.534 75.316) (end 95.384 75.316) (width 0.254) (layer "F.Cu") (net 5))
 (segment (start 90.604 51.776) (end 78.154 64.226) (width 0.254) (layer "F.Cu") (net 2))
 (segment (start 93.464 51.776) (end 90.604 51.776) (width 0.254) (layer "F.Cu") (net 2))
 (segment (start 80.694 79.466) (end 83.194 81.966) (width 0.254) (layer "F.Cu") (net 15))
 (segment (start 83.194 81.966) (end 99.034 81.966) (width 0.254) (layer "F.Cu") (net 15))
 (segment (start 99.034 81.966) (end 111.534 81.966) (width 0.254) (layer "F.Cu") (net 15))
 (segment (start 114.141 78.323) (end 117.784 81.966) (width 0.254) (layer "F.Cu") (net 14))
 (segment (start 83.234 79.466) (end 84.377 78.323) (width 0.254) (layer "F.Cu") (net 14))
 (segment (start 84.377 78.323) (end 114.141 78.323) (width 0.254) (layer "F.Cu") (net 14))
 (segment (start 117.784 81.966) (end 130.284 81.966) (width 0.254) (layer "F.Cu") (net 14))
 (segment (start 70.604 44.156) (end 70.604 50.035103) (width 0.254) (layer "F.Cu") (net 4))
 (segment (start 69.373 63.065) (end 70.534 64.226) (width 0.254) (layer "F.Cu") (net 4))
 (segment (start 69.373 51.266103) (end 69.373 63.065) (width 0.254) (layer "F.Cu") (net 4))
 (segment (start 70.604 50.035103) (end 69.373 51.266103) (width 0.254) (layer "F.Cu") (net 4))
 (segment (start 119 66) (end 119.034 65.966) (width 0.5) (layer "F.Cu") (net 7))
 (segment (start 69.268 76.732) (end 80 66) (width 0.5) (layer "F.Cu") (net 7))
 (segment (start 80 66) (end 119 66) (width 0.5) (layer "F.Cu") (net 7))
 (segment (start 69.268 84.7) (end 69.268 76.732) (width 0.5) (layer "F.Cu") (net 7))
 (segment (start 74.034 89.466) (end 69.268 84.7) (width 0.5) (layer "F.Cu") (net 7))
 (segment (start 121.484 68.416) (end 121.534 68.416) (width 0.5) (layer "F.Cu") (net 7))
 (segment (start 119.034 65.966) (end 121.484 68.416) (width 0.5) (layer "F.Cu") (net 7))
 (segment (start 93.464 46.376) (end 75.614 64.226) (width 0.254) (layer "F.Cu") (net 1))
 (segment (start 75.614 64.186) (end 75.614 64.226) (width 0.254) (layer "F.Cu") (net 1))
 (segment (start 93.464 44.156) (end 93.464 46.376) (width 0.254) (layer "F.Cu") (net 1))
 (segment (start 70.604 61.756) (end 73.074 64.226) (width 0.254) (layer "F.Cu") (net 3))
 (segment (start 70.604 51.776) (end 70.604 61.756) (width 0.254) (layer "F.Cu") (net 3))
 (segment (start 80.654 76.966) (end 78.154 79.466) (width 0.254) (layer "F.Cu") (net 6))
 (segment (start 91.534 76.966) (end 80.654 76.966) (width 0.254) (layer "F.Cu") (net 6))
 (segment (start 75.614 79.466) (end 76.537553 79.466) (width 0.254) (layer "B.Cu") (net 9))
 (segment (start 75.614 79.466) (end 114.454 40.626) (width 0.5) (layer "B.Cu") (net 9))
 (segment (start 114.454 40.626) (end 114.454 36.466) (width 0.5) (layer "B.Cu") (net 9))
 (segment (start 76.534 89.466) (end 76.534 85.466) (width 0.5) (layer "F.Cu") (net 13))
 (segment (start 76.534 85.466) (end 70.534 79.466) (width 0.5) (layer "F.Cu") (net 13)))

